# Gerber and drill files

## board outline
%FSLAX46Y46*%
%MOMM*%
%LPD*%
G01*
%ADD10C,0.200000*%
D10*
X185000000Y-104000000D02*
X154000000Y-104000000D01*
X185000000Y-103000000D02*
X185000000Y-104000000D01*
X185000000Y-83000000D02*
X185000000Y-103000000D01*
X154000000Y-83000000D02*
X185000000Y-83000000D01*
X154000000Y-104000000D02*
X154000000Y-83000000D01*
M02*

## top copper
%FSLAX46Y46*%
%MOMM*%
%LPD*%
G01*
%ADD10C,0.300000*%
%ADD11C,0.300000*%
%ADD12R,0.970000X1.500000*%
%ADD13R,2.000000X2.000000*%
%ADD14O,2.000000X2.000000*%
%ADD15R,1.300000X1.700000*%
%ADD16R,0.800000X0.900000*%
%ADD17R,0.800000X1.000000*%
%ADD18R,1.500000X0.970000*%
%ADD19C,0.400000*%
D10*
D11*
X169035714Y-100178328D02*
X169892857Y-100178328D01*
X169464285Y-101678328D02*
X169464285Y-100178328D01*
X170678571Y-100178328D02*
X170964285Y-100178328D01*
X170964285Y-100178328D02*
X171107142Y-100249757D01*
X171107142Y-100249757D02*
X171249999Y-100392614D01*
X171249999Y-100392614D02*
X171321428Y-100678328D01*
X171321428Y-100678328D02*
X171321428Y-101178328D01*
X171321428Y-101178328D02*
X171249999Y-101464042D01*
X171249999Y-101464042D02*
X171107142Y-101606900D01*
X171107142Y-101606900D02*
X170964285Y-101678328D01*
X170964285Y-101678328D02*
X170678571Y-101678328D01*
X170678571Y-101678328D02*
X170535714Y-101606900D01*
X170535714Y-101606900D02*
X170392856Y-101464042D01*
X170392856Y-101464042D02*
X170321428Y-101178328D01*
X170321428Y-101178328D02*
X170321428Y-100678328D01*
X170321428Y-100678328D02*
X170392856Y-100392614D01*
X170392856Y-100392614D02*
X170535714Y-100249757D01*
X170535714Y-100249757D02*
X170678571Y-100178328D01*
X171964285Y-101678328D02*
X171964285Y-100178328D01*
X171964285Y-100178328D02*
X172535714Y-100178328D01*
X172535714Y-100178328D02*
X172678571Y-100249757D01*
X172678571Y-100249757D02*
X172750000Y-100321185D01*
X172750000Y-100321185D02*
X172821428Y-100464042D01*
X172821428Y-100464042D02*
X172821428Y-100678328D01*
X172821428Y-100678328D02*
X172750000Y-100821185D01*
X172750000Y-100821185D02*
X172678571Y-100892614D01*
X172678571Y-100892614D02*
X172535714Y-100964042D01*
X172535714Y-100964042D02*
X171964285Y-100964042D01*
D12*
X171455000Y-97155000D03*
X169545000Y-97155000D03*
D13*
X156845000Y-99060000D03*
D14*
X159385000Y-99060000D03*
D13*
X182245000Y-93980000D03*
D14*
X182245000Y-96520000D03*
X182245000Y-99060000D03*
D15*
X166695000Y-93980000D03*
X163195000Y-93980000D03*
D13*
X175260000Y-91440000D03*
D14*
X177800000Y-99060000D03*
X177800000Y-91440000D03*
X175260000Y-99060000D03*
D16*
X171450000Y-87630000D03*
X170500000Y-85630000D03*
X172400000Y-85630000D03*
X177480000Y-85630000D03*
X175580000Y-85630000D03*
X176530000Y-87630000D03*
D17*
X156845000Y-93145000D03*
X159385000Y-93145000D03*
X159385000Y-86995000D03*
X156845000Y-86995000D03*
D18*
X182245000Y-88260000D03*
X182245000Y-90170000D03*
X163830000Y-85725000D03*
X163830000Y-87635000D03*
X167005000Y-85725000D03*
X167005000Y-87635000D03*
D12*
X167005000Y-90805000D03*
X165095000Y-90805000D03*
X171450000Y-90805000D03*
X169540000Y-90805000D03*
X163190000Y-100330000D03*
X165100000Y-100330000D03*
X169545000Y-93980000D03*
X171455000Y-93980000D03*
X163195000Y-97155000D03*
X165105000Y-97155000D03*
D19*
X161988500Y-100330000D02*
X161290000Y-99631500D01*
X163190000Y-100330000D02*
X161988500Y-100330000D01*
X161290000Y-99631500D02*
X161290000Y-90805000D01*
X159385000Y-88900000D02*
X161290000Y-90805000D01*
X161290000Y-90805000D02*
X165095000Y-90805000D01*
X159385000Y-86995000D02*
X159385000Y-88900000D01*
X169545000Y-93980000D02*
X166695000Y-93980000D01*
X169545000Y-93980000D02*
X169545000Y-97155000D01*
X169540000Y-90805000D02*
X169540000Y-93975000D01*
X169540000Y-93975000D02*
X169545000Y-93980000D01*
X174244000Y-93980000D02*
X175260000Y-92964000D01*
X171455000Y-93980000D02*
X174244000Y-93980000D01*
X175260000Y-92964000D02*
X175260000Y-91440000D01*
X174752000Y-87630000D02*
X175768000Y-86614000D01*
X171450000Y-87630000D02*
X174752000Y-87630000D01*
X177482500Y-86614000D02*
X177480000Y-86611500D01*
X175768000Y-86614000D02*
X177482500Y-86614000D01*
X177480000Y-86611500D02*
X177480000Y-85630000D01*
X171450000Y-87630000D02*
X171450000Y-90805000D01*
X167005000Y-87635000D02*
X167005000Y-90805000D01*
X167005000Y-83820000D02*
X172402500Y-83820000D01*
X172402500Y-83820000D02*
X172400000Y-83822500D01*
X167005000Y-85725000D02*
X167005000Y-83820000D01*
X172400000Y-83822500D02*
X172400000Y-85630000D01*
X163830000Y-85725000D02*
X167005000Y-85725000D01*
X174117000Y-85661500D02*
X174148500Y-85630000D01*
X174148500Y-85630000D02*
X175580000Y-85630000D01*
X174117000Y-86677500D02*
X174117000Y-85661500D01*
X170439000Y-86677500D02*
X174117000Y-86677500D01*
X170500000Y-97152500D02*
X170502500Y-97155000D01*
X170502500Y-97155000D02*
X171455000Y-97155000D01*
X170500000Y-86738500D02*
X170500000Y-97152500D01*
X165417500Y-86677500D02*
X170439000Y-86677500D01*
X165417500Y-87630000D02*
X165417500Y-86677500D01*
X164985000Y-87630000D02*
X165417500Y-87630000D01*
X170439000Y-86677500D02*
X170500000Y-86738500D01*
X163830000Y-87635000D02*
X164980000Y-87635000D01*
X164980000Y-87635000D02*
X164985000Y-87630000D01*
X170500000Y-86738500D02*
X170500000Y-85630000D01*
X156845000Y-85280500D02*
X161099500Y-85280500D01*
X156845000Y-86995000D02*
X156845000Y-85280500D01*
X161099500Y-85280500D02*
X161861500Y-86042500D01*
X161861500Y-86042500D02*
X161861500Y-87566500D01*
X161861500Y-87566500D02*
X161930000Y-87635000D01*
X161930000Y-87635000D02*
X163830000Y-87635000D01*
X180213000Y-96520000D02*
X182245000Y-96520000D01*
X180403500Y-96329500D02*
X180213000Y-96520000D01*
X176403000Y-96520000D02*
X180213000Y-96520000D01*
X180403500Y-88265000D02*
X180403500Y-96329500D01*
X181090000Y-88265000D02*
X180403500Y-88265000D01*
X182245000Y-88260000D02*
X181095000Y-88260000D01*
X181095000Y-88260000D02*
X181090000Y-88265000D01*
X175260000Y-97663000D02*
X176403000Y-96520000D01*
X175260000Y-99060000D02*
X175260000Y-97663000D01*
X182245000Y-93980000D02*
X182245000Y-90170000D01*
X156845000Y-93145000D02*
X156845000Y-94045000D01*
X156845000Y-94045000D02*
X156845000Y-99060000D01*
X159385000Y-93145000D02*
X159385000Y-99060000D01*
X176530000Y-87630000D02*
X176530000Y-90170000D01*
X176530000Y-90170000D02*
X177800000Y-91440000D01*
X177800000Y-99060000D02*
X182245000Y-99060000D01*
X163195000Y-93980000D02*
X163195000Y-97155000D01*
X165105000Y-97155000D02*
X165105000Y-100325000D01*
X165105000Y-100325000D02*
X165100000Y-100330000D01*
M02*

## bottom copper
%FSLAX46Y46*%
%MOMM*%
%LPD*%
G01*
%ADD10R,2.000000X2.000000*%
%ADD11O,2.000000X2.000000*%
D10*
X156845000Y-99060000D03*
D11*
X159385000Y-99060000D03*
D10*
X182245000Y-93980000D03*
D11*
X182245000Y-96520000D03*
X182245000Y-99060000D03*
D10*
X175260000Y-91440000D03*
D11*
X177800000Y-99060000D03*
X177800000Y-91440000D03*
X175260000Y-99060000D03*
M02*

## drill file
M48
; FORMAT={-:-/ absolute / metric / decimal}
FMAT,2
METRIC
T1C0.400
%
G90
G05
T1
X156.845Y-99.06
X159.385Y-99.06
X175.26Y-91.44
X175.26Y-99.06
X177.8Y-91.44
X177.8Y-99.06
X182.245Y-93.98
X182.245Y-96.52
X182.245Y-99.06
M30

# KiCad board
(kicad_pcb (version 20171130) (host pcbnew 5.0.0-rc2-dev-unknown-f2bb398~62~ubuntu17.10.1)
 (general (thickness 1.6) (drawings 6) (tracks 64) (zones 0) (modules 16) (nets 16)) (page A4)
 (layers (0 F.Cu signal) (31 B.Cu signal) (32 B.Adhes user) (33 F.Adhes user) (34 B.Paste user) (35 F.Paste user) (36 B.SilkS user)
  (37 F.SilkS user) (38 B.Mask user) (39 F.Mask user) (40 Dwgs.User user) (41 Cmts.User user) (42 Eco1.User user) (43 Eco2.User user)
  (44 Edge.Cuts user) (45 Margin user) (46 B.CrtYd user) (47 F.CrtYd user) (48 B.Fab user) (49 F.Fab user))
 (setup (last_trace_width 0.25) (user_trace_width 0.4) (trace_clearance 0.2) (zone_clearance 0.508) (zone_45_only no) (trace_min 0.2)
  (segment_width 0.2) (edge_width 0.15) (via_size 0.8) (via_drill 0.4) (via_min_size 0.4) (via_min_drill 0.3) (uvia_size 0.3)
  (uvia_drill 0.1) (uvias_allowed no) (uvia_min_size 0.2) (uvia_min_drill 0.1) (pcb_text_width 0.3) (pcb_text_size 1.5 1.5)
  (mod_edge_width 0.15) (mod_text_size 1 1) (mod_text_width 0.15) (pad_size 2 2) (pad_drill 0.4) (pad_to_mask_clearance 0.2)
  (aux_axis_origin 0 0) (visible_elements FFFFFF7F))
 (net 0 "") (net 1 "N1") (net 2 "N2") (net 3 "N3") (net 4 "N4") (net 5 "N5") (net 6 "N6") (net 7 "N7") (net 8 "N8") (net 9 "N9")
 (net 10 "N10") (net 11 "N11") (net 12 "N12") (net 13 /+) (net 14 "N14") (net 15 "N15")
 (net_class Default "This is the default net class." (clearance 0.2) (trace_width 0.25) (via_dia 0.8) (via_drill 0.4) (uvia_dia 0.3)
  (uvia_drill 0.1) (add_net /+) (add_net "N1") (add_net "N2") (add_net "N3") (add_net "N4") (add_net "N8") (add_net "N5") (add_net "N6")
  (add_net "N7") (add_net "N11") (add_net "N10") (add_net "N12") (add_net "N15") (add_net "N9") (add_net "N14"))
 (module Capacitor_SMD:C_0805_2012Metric (layer F.Cu) (at 170.5 97.155 180)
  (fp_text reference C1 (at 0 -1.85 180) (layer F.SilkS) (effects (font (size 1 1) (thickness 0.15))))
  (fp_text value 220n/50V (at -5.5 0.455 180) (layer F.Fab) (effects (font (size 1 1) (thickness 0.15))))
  (pad 1 smd rect (at -0.955 0 180) (size 0.97 1.5) (layers F.Cu F.Paste F.Mask) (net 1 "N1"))
  (pad 2 smd rect (at 0.955 0 180) (size 0.97 1.5) (layers F.Cu F.Paste F.Mask) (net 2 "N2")))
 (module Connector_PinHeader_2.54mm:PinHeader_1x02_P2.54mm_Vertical (layer B.Cu) (at 156.845 99.06 270)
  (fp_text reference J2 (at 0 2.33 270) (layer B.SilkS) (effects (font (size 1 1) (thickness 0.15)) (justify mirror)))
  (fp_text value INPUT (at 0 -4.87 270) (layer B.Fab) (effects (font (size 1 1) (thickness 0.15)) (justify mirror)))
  (pad 1 thru_hole rect (at 0 0 270) (size 2 2) (drill 0.4) (layers *.Cu *.Mask) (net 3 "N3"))
  (pad 2 thru_hole oval (at 0 -2.54 270) (size 2 2) (drill 0.4) (layers *.Cu *.Mask) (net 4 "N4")))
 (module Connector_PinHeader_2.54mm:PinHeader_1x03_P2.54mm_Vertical (layer B.Cu) (at 182.245 93.98 180)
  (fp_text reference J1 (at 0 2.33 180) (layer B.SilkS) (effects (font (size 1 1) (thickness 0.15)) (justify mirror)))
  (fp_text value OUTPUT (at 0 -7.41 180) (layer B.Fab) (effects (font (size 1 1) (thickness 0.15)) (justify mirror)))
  (pad 1 thru_hole rect (at 0 0 180) (size 2 2) (drill 0.4) (layers *.Cu *.Mask) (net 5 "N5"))
  (pad 2 thru_hole oval (at 0 -2.54 180) (size 2 2) (drill 0.4) (layers *.Cu *.Mask) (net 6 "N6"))
  (pad 3 thru_hole oval (at 0 -5.08 180) (size 2 2) (drill 0.4) (layers *.Cu *.Mask) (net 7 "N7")))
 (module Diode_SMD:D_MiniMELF (layer F.Cu) (at 164.945 93.98 180)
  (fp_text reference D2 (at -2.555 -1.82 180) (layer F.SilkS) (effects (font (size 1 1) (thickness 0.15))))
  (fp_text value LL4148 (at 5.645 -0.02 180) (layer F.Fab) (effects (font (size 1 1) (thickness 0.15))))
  (pad 1 smd rect (at -1.75 0 180) (size 1.3 1.7) (layers F.Cu F.Paste F.Mask) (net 2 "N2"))
  (pad 2 smd rect (at 1.75 0 180) (size 1.3 1.7) (layers F.Cu F.Paste F.Mask) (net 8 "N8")))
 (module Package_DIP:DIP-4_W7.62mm (layer B.Cu) (at 175.26 91.44 270)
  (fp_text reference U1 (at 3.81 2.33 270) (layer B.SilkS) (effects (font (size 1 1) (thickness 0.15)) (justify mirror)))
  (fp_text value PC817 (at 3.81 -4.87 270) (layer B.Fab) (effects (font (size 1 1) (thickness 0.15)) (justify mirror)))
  (pad 1 thru_hole rect (at 0 0 270) (size 2 2) (drill 0.4) (layers *.Cu *.Mask) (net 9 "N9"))
  (pad 3 thru_hole oval (at 7.62 -2.54 270) (size 2 2) (drill 0.4) (layers *.Cu *.Mask) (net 7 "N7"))
  (pad 2 thru_hole oval (at 0 -2.54 270) (size 2 2) (drill 0.4) (layers *.Cu *.Mask) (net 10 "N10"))
  (pad 4 thru_hole oval (at 7.62 0 270) (size 2 2) (drill 0.4) (layers *.Cu *.Mask) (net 6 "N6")))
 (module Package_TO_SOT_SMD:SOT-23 (layer F.Cu) (at 171.45 86.63 270)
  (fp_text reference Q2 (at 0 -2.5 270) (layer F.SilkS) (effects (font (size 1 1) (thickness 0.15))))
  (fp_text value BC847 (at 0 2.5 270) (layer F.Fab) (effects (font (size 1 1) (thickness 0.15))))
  (pad 3 smd rect (at 1 0 270) (size 0.9 0.8) (layers F.Cu F.Paste F.Mask) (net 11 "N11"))
  (pad 2 smd rect (at -1 0.95 270) (size 0.9 0.8) (layers F.Cu F.Paste F.Mask) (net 1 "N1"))
  (pad 1 smd rect (at -1 -0.95 270) (size 0.9 0.8) (layers F.Cu F.Paste F.Mask) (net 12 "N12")))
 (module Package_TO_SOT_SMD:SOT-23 (layer F.Cu) (at 176.53 86.63 270)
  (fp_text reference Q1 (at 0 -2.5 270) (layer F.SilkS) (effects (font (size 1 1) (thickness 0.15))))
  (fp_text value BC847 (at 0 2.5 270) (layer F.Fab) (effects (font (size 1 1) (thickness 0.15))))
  (pad 1 smd rect (at -1 -0.95 270) (size 0.9 0.8) (layers F.Cu F.Paste F.Mask) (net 11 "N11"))
  (pad 2 smd rect (at -1 0.95 270) (size 0.9 0.8) (layers F.Cu F.Paste F.Mask) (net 1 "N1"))
  (pad 3 smd rect (at 1 0 270) (size 0.9 0.8) (layers F.Cu F.Paste F.Mask) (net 10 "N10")))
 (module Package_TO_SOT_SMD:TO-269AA (layer F.Cu) (at 158.115 90.07 90)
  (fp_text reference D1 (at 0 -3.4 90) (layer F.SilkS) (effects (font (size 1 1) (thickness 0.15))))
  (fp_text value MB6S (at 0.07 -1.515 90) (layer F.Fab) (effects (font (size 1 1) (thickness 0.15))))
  (pad 1 smd rect (at -3.075 -1.27 90) (size 1 0.8) (layers F.Cu F.Paste F.Mask) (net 3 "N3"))
  (pad 2 smd rect (at -3.075 1.27 90) (size 1 0.8) (layers F.Cu F.Paste F.Mask) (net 4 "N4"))
  (pad 3 smd rect (at 3.075 1.27 90) (size 1 0.8) (layers F.Cu F.Paste F.Mask) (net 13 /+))
  (pad 4 smd rect (at 3.075 -1.27 90) (size 1 0.8) (layers F.Cu F.Paste F.Mask) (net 1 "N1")))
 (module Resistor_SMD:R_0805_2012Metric (layer F.Cu) (at 182.245 89.215 90)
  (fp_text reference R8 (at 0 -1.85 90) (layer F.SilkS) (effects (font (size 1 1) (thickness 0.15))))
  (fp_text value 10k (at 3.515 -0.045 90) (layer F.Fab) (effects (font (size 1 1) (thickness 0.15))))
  (pad 2 smd rect (at 0.955 0 90) (size 0.97 1.5) (layers F.Cu F.Paste F.Mask) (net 6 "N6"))
  (pad 1 smd rect (at -0.955 0 90) (size 0.97 1.5) (layers F.Cu F.Paste F.Mask) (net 5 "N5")))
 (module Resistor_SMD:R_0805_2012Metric (layer F.Cu) (at 163.83 86.68 270)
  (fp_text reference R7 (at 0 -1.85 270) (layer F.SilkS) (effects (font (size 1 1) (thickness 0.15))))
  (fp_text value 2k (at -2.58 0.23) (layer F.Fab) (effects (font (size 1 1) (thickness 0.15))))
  (pad 1 smd rect (at -0.955 0 270) (size 0.97 1.5) (layers F.Cu F.Paste F.Mask) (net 12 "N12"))
  (pad 2 smd rect (at 0.955 0 270) (size 0.97 1.5) (layers F.Cu F.Paste F.Mask) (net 1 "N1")))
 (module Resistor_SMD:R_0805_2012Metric (layer F.Cu) (at 167.005 86.68 90)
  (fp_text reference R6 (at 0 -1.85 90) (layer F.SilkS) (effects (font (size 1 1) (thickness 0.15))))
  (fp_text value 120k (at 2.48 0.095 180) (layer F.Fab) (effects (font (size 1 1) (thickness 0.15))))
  (pad 2 smd rect (at 0.955 0 90) (size 0.97 1.5) (layers F.Cu F.Paste F.Mask) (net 12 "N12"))
  (pad 1 smd rect (at -0.955 0 90) (size 0.97 1.5) (layers F.Cu F.Paste F.Mask) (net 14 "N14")))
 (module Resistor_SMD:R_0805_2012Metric (layer F.Cu) (at 166.05 90.805 180)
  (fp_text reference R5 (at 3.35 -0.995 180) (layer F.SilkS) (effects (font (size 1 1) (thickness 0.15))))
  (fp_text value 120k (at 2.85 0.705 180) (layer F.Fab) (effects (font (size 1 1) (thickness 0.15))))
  (pad 1 smd rect (at -0.955 0 180) (size 0.97 1.5) (layers F.Cu F.Paste F.Mask) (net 14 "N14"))
  (pad 2 smd rect (at 0.955 0 180) (size 0.97 1.5) (layers F.Cu F.Paste F.Mask) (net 13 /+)))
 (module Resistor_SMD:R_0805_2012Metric (layer F.Cu) (at 170.495 90.805)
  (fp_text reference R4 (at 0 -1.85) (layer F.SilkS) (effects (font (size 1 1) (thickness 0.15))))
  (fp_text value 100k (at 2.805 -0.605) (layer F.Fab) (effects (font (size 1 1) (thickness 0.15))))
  (pad 2 smd rect (at 0.955 0) (size 0.97 1.5) (layers F.Cu F.Paste F.Mask) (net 11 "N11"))
  (pad 1 smd rect (at -0.955 0) (size 0.97 1.5) (layers F.Cu F.Paste F.Mask) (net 2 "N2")))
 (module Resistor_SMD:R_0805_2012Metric (layer F.Cu) (at 164.145 100.33)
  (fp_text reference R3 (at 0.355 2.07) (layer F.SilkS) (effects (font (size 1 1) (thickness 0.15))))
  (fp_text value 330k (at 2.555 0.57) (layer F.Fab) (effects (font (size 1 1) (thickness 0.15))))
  (pad 1 smd rect (at -0.955 0) (size 0.97 1.5) (layers F.Cu F.Paste F.Mask) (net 13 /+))
  (pad 2 smd rect (at 0.955 0) (size 0.97 1.5) (layers F.Cu F.Paste F.Mask) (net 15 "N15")))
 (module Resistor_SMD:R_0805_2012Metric (layer F.Cu) (at 170.5 93.98 180)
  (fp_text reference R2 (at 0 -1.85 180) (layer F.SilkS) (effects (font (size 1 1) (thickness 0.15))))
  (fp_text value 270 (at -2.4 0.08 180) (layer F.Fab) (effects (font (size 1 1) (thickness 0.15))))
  (pad 2 smd rect (at 0.955 0 180) (size 0.97 1.5) (layers F.Cu F.Paste F.Mask) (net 2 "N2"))
  (pad 1 smd rect (at -0.955 0 180) (size 0.97 1.5) (layers F.Cu F.Paste F.Mask) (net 9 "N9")))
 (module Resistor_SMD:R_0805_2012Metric (layer F.Cu) (at 164.15 97.155)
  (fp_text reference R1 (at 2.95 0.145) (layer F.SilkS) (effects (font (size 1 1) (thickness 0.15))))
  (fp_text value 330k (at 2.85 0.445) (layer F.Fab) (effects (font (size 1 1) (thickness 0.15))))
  (pad 1 smd rect (at -0.955 0) (size 0.97 1.5) (layers F.Cu F.Paste F.Mask) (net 8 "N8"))
  (pad 2 smd rect (at 0.955 0) (size 0.97 1.5) (layers F.Cu F.Paste F.Mask) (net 15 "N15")))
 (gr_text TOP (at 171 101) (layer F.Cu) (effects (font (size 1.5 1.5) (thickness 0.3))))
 (gr_line (start 185 104) (end 154 104) (layer Edge.Cuts) (width 0.2))
 (gr_line (start 185 103) (end 185 104) (layer Edge.Cuts) (width 0.2))
 (gr_line (start 185 83) (end 185 103) (layer Edge.Cuts) (width 0.2))
 (gr_line (start 154 83) (end 185 83) (layer Edge.Cuts) (width 0.2))
 (gr_line (start 154 104) (end 154 83) (layer Edge.Cuts) (width 0.2))
 (segment (start 161.9885 100.33) (end 161.29 99.6315) (width 0.4) (layer F.Cu) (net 13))
 (segment (start 163.19 100.33) (end 161.9885 100.33) (width 0.4) (layer F.Cu) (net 13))
 (segment (start 161.29 99.6315) (end 161.29 90.805) (width 0.4) (layer F.Cu) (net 13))
 (segment (start 159.385 88.9) (end 161.29 90.805) (width 0.4) (layer F.Cu) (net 13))
 (segment (start 161.29 90.805) (end 165.095 90.805) (width 0.4) (layer F.Cu) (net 13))
 (segment (start 159.385 86.995) (end 159.385 88.9) (width 0.4) (layer F.Cu) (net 13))
 (segment (start 169.545 93.98) (end 166.695 93.98) (width 0.4) (layer F.Cu) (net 2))
 (segment (start 169.545 93.98) (end 169.545 97.155) (width 0.4) (layer F.Cu) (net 2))
 (segment (start 169.54 90.805) (end 169.54 93.975) (width 0.4) (layer F.Cu) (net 2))
 (segment (start 169.54 93.975) (end 169.545 93.98) (width 0.4) (layer F.Cu) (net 2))
 (segment (start 174.244 93.98) (end 175.26 92.964) (width 0.4) (layer F.Cu) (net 9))
 (segment (start 171.455 93.98) (end 174.244 93.98) (width 0.4) (layer F.Cu) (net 9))
 (segment (start 175.26 92.964) (end 175.26 91.44) (width 0.4) (layer F.Cu) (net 9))
 (segment (start 174.752 87.63) (end 175.768 86.614) (width 0.4) (layer F.Cu) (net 11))
 (segment (start 171.45 87.63) (end 174.752 87.63) (width 0.4) (layer F.Cu) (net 11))
 (segment (start 177.4825 86.614) (end 177.48 86.6115) (width 0.4) (layer F.Cu) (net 11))
 (segment (start 175.768 86.614) (end 177.4825 86.614) (width 0.4) (layer F.Cu) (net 11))
 (segment (start 177.48 86.6115) (end 177.48 85.63) (width 0.4) (layer F.Cu) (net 11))
 (segment (start 171.45 87.63) (end 171.45 90.805) (width 0.4) (layer F.Cu) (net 11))
 (segment (start 167.005 87.635) (end 167.005 90.805) (width 0.4) (layer F.Cu) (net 14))
 (segment (start 167.005 83.82) (end 172.4025 83.82) (width 0.4) (layer F.Cu) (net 12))
 (segment (start 172.4025 83.82) (end 172.4 83.8225) (width 0.4) (layer F.Cu) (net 12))
 (segment (start 167.005 85.725) (end 167.005 83.82) (width 0.4) (layer F.Cu) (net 12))
 (segment (start 172.4 83.8225) (end 172.4 85.63) (width 0.4) (layer F.Cu) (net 12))
 (segment (start 163.83 85.725) (end 167.005 85.725) (width 0.4) (layer F.Cu) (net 12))
 (segment (start 174.117 85.6615) (end 174.1485 85.63) (width 0.4) (layer F.Cu) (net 1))
 (segment (start 174.1485 85.63) (end 175.58 85.63) (width 0.4) (layer F.Cu) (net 1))
 (segment (start 174.117 86.6775) (end 174.117 85.6615) (width 0.4) (layer F.Cu) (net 1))
 (segment (start 170.439 86.6775) (end 174.117 86.6775) (width 0.4) (layer F.Cu) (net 1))
 (segment (start 170.5 97.1525) (end 170.5025 97.155) (width 0.4) (layer F.Cu) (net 1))
 (segment (start 170.5025 97.155) (end 171.455 97.155) (width 0.4) (layer F.Cu) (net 1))
 (segment (start 170.5 86.7385) (end 170.5 97.1525) (width 0.4) (layer F.Cu) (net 1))
 (segment (start 165.4175 86.6775) (end 170.439 86.6775) (width 0.4) (layer F.Cu) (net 1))
 (segment (start 165.4175 87.63) (end 165.4175 86.6775) (width 0.4) (layer F.Cu) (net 1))
 (segment (start 164.985 87.63) (end 165.4175 87.63) (width 0.4) (layer F.Cu) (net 1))
 (segment (start 170.439 86.6775) (end 170.5 86.7385) (width 0.4) (layer F.Cu) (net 1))
 (segment (start 163.83 87.635) (end 164.98 87.635) (width 0.4) (layer F.Cu) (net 1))
 (segment (start 164.98 87.635) (end 164.985 87.63) (width 0.4) (layer F.Cu) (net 1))
 (segment (start 170.5 86.7385) (end 170.5 85.63) (width 0.4) (layer F.Cu) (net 1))
 (segment (start 156.845 85.2805) (end 161.0995 85.2805) (width 0.4) (layer F.Cu) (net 1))
 (segment (start 156.845 86.995) (end 156.845 85.2805) (width 0.4) (layer F.Cu) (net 1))
 (segment (start 161.0995 85.2805) (end 161.8615 86.0425) (width 0.4) (layer F.Cu) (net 1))
 (segment (start 161.8615 86.0425) (end 161.8615 87.5665) (width 0.4) (layer F.Cu) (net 1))
 (segment (start 161.8615 87.5665) (end 161.93 87.635) (width 0.4) (layer F.Cu) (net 1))
 (segment (start 161.93 87.635) (end 163.83 87.635) (width 0.4) (layer F.Cu) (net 1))
 (segment (start 180.213 96.52) (end 182.245 96.52) (width 0.4) (layer F.Cu) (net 6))
 (segment (start 180.4035 96.3295) (end 180.213 96.52) (width 0.4) (layer F.Cu) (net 6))
 (segment (start 176.403 96.52) (end 180.213 96.52) (width 0.4) (layer F.Cu) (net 6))
 (segment (start 180.4035 88.265) (end 180.4035 96.3295) (width 0.4) (layer F.Cu) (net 6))
 (segment (start 181.09 88.265) (end 180.4035 88.265) (width 0.4) (layer F.Cu) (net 6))
 (segment (start 182.245 88.26) (end 181.095 88.26) (width 0.4) (layer F.Cu) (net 6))
 (segment (start 181.095 88.26) (end 181.09 88.265) (width 0.4) (layer F.Cu) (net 6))
 (segment (start 175.26 97.663) (end 176.403 96.52) (width 0.4) (layer F.Cu) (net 6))
 (segment (start 175.26 99.06) (end 175.26 97.663) (width 0.4) (layer F.Cu) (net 6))
 (segment (start 182.245 93.98) (end 182.245 90.17) (width 0.4) (layer F.Cu) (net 5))
 (segment (start 156.845 93.145) (end 156.845 94.045) (width 0.4) (layer F.Cu) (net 3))
 (segment (start 156.845 94.045) (end 156.845 99.06) (width 0.4) (layer F.Cu) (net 3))
 (segment (start 159.385 93.145) (end 159.385 99.06) (width 0.4) (layer F.Cu) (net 4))
 (segment (start 176.53 87.63) (end 176.53 90.17) (width 0.4) (layer F.Cu) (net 10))
 (segment (start 176.53 90.17) (end 177.8 91.44) (width 0.4) (layer F.Cu) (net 10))
 (segment (start 177.8 99.06) (end 182.245 99.06) (width 0.4) (layer F.Cu) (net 7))
 (segment (start 163.195 93.98) (end 163.195 97.155) (width 0.4) (layer F.Cu) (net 8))
 (segment (start 165.105 97.155) (end 165.105 100.325) (width 0.4) (layer F.Cu) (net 15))
 (segment (start 165.105 100.325) (end 165.1 100.33) (width 0.4) (layer F.Cu) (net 15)))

